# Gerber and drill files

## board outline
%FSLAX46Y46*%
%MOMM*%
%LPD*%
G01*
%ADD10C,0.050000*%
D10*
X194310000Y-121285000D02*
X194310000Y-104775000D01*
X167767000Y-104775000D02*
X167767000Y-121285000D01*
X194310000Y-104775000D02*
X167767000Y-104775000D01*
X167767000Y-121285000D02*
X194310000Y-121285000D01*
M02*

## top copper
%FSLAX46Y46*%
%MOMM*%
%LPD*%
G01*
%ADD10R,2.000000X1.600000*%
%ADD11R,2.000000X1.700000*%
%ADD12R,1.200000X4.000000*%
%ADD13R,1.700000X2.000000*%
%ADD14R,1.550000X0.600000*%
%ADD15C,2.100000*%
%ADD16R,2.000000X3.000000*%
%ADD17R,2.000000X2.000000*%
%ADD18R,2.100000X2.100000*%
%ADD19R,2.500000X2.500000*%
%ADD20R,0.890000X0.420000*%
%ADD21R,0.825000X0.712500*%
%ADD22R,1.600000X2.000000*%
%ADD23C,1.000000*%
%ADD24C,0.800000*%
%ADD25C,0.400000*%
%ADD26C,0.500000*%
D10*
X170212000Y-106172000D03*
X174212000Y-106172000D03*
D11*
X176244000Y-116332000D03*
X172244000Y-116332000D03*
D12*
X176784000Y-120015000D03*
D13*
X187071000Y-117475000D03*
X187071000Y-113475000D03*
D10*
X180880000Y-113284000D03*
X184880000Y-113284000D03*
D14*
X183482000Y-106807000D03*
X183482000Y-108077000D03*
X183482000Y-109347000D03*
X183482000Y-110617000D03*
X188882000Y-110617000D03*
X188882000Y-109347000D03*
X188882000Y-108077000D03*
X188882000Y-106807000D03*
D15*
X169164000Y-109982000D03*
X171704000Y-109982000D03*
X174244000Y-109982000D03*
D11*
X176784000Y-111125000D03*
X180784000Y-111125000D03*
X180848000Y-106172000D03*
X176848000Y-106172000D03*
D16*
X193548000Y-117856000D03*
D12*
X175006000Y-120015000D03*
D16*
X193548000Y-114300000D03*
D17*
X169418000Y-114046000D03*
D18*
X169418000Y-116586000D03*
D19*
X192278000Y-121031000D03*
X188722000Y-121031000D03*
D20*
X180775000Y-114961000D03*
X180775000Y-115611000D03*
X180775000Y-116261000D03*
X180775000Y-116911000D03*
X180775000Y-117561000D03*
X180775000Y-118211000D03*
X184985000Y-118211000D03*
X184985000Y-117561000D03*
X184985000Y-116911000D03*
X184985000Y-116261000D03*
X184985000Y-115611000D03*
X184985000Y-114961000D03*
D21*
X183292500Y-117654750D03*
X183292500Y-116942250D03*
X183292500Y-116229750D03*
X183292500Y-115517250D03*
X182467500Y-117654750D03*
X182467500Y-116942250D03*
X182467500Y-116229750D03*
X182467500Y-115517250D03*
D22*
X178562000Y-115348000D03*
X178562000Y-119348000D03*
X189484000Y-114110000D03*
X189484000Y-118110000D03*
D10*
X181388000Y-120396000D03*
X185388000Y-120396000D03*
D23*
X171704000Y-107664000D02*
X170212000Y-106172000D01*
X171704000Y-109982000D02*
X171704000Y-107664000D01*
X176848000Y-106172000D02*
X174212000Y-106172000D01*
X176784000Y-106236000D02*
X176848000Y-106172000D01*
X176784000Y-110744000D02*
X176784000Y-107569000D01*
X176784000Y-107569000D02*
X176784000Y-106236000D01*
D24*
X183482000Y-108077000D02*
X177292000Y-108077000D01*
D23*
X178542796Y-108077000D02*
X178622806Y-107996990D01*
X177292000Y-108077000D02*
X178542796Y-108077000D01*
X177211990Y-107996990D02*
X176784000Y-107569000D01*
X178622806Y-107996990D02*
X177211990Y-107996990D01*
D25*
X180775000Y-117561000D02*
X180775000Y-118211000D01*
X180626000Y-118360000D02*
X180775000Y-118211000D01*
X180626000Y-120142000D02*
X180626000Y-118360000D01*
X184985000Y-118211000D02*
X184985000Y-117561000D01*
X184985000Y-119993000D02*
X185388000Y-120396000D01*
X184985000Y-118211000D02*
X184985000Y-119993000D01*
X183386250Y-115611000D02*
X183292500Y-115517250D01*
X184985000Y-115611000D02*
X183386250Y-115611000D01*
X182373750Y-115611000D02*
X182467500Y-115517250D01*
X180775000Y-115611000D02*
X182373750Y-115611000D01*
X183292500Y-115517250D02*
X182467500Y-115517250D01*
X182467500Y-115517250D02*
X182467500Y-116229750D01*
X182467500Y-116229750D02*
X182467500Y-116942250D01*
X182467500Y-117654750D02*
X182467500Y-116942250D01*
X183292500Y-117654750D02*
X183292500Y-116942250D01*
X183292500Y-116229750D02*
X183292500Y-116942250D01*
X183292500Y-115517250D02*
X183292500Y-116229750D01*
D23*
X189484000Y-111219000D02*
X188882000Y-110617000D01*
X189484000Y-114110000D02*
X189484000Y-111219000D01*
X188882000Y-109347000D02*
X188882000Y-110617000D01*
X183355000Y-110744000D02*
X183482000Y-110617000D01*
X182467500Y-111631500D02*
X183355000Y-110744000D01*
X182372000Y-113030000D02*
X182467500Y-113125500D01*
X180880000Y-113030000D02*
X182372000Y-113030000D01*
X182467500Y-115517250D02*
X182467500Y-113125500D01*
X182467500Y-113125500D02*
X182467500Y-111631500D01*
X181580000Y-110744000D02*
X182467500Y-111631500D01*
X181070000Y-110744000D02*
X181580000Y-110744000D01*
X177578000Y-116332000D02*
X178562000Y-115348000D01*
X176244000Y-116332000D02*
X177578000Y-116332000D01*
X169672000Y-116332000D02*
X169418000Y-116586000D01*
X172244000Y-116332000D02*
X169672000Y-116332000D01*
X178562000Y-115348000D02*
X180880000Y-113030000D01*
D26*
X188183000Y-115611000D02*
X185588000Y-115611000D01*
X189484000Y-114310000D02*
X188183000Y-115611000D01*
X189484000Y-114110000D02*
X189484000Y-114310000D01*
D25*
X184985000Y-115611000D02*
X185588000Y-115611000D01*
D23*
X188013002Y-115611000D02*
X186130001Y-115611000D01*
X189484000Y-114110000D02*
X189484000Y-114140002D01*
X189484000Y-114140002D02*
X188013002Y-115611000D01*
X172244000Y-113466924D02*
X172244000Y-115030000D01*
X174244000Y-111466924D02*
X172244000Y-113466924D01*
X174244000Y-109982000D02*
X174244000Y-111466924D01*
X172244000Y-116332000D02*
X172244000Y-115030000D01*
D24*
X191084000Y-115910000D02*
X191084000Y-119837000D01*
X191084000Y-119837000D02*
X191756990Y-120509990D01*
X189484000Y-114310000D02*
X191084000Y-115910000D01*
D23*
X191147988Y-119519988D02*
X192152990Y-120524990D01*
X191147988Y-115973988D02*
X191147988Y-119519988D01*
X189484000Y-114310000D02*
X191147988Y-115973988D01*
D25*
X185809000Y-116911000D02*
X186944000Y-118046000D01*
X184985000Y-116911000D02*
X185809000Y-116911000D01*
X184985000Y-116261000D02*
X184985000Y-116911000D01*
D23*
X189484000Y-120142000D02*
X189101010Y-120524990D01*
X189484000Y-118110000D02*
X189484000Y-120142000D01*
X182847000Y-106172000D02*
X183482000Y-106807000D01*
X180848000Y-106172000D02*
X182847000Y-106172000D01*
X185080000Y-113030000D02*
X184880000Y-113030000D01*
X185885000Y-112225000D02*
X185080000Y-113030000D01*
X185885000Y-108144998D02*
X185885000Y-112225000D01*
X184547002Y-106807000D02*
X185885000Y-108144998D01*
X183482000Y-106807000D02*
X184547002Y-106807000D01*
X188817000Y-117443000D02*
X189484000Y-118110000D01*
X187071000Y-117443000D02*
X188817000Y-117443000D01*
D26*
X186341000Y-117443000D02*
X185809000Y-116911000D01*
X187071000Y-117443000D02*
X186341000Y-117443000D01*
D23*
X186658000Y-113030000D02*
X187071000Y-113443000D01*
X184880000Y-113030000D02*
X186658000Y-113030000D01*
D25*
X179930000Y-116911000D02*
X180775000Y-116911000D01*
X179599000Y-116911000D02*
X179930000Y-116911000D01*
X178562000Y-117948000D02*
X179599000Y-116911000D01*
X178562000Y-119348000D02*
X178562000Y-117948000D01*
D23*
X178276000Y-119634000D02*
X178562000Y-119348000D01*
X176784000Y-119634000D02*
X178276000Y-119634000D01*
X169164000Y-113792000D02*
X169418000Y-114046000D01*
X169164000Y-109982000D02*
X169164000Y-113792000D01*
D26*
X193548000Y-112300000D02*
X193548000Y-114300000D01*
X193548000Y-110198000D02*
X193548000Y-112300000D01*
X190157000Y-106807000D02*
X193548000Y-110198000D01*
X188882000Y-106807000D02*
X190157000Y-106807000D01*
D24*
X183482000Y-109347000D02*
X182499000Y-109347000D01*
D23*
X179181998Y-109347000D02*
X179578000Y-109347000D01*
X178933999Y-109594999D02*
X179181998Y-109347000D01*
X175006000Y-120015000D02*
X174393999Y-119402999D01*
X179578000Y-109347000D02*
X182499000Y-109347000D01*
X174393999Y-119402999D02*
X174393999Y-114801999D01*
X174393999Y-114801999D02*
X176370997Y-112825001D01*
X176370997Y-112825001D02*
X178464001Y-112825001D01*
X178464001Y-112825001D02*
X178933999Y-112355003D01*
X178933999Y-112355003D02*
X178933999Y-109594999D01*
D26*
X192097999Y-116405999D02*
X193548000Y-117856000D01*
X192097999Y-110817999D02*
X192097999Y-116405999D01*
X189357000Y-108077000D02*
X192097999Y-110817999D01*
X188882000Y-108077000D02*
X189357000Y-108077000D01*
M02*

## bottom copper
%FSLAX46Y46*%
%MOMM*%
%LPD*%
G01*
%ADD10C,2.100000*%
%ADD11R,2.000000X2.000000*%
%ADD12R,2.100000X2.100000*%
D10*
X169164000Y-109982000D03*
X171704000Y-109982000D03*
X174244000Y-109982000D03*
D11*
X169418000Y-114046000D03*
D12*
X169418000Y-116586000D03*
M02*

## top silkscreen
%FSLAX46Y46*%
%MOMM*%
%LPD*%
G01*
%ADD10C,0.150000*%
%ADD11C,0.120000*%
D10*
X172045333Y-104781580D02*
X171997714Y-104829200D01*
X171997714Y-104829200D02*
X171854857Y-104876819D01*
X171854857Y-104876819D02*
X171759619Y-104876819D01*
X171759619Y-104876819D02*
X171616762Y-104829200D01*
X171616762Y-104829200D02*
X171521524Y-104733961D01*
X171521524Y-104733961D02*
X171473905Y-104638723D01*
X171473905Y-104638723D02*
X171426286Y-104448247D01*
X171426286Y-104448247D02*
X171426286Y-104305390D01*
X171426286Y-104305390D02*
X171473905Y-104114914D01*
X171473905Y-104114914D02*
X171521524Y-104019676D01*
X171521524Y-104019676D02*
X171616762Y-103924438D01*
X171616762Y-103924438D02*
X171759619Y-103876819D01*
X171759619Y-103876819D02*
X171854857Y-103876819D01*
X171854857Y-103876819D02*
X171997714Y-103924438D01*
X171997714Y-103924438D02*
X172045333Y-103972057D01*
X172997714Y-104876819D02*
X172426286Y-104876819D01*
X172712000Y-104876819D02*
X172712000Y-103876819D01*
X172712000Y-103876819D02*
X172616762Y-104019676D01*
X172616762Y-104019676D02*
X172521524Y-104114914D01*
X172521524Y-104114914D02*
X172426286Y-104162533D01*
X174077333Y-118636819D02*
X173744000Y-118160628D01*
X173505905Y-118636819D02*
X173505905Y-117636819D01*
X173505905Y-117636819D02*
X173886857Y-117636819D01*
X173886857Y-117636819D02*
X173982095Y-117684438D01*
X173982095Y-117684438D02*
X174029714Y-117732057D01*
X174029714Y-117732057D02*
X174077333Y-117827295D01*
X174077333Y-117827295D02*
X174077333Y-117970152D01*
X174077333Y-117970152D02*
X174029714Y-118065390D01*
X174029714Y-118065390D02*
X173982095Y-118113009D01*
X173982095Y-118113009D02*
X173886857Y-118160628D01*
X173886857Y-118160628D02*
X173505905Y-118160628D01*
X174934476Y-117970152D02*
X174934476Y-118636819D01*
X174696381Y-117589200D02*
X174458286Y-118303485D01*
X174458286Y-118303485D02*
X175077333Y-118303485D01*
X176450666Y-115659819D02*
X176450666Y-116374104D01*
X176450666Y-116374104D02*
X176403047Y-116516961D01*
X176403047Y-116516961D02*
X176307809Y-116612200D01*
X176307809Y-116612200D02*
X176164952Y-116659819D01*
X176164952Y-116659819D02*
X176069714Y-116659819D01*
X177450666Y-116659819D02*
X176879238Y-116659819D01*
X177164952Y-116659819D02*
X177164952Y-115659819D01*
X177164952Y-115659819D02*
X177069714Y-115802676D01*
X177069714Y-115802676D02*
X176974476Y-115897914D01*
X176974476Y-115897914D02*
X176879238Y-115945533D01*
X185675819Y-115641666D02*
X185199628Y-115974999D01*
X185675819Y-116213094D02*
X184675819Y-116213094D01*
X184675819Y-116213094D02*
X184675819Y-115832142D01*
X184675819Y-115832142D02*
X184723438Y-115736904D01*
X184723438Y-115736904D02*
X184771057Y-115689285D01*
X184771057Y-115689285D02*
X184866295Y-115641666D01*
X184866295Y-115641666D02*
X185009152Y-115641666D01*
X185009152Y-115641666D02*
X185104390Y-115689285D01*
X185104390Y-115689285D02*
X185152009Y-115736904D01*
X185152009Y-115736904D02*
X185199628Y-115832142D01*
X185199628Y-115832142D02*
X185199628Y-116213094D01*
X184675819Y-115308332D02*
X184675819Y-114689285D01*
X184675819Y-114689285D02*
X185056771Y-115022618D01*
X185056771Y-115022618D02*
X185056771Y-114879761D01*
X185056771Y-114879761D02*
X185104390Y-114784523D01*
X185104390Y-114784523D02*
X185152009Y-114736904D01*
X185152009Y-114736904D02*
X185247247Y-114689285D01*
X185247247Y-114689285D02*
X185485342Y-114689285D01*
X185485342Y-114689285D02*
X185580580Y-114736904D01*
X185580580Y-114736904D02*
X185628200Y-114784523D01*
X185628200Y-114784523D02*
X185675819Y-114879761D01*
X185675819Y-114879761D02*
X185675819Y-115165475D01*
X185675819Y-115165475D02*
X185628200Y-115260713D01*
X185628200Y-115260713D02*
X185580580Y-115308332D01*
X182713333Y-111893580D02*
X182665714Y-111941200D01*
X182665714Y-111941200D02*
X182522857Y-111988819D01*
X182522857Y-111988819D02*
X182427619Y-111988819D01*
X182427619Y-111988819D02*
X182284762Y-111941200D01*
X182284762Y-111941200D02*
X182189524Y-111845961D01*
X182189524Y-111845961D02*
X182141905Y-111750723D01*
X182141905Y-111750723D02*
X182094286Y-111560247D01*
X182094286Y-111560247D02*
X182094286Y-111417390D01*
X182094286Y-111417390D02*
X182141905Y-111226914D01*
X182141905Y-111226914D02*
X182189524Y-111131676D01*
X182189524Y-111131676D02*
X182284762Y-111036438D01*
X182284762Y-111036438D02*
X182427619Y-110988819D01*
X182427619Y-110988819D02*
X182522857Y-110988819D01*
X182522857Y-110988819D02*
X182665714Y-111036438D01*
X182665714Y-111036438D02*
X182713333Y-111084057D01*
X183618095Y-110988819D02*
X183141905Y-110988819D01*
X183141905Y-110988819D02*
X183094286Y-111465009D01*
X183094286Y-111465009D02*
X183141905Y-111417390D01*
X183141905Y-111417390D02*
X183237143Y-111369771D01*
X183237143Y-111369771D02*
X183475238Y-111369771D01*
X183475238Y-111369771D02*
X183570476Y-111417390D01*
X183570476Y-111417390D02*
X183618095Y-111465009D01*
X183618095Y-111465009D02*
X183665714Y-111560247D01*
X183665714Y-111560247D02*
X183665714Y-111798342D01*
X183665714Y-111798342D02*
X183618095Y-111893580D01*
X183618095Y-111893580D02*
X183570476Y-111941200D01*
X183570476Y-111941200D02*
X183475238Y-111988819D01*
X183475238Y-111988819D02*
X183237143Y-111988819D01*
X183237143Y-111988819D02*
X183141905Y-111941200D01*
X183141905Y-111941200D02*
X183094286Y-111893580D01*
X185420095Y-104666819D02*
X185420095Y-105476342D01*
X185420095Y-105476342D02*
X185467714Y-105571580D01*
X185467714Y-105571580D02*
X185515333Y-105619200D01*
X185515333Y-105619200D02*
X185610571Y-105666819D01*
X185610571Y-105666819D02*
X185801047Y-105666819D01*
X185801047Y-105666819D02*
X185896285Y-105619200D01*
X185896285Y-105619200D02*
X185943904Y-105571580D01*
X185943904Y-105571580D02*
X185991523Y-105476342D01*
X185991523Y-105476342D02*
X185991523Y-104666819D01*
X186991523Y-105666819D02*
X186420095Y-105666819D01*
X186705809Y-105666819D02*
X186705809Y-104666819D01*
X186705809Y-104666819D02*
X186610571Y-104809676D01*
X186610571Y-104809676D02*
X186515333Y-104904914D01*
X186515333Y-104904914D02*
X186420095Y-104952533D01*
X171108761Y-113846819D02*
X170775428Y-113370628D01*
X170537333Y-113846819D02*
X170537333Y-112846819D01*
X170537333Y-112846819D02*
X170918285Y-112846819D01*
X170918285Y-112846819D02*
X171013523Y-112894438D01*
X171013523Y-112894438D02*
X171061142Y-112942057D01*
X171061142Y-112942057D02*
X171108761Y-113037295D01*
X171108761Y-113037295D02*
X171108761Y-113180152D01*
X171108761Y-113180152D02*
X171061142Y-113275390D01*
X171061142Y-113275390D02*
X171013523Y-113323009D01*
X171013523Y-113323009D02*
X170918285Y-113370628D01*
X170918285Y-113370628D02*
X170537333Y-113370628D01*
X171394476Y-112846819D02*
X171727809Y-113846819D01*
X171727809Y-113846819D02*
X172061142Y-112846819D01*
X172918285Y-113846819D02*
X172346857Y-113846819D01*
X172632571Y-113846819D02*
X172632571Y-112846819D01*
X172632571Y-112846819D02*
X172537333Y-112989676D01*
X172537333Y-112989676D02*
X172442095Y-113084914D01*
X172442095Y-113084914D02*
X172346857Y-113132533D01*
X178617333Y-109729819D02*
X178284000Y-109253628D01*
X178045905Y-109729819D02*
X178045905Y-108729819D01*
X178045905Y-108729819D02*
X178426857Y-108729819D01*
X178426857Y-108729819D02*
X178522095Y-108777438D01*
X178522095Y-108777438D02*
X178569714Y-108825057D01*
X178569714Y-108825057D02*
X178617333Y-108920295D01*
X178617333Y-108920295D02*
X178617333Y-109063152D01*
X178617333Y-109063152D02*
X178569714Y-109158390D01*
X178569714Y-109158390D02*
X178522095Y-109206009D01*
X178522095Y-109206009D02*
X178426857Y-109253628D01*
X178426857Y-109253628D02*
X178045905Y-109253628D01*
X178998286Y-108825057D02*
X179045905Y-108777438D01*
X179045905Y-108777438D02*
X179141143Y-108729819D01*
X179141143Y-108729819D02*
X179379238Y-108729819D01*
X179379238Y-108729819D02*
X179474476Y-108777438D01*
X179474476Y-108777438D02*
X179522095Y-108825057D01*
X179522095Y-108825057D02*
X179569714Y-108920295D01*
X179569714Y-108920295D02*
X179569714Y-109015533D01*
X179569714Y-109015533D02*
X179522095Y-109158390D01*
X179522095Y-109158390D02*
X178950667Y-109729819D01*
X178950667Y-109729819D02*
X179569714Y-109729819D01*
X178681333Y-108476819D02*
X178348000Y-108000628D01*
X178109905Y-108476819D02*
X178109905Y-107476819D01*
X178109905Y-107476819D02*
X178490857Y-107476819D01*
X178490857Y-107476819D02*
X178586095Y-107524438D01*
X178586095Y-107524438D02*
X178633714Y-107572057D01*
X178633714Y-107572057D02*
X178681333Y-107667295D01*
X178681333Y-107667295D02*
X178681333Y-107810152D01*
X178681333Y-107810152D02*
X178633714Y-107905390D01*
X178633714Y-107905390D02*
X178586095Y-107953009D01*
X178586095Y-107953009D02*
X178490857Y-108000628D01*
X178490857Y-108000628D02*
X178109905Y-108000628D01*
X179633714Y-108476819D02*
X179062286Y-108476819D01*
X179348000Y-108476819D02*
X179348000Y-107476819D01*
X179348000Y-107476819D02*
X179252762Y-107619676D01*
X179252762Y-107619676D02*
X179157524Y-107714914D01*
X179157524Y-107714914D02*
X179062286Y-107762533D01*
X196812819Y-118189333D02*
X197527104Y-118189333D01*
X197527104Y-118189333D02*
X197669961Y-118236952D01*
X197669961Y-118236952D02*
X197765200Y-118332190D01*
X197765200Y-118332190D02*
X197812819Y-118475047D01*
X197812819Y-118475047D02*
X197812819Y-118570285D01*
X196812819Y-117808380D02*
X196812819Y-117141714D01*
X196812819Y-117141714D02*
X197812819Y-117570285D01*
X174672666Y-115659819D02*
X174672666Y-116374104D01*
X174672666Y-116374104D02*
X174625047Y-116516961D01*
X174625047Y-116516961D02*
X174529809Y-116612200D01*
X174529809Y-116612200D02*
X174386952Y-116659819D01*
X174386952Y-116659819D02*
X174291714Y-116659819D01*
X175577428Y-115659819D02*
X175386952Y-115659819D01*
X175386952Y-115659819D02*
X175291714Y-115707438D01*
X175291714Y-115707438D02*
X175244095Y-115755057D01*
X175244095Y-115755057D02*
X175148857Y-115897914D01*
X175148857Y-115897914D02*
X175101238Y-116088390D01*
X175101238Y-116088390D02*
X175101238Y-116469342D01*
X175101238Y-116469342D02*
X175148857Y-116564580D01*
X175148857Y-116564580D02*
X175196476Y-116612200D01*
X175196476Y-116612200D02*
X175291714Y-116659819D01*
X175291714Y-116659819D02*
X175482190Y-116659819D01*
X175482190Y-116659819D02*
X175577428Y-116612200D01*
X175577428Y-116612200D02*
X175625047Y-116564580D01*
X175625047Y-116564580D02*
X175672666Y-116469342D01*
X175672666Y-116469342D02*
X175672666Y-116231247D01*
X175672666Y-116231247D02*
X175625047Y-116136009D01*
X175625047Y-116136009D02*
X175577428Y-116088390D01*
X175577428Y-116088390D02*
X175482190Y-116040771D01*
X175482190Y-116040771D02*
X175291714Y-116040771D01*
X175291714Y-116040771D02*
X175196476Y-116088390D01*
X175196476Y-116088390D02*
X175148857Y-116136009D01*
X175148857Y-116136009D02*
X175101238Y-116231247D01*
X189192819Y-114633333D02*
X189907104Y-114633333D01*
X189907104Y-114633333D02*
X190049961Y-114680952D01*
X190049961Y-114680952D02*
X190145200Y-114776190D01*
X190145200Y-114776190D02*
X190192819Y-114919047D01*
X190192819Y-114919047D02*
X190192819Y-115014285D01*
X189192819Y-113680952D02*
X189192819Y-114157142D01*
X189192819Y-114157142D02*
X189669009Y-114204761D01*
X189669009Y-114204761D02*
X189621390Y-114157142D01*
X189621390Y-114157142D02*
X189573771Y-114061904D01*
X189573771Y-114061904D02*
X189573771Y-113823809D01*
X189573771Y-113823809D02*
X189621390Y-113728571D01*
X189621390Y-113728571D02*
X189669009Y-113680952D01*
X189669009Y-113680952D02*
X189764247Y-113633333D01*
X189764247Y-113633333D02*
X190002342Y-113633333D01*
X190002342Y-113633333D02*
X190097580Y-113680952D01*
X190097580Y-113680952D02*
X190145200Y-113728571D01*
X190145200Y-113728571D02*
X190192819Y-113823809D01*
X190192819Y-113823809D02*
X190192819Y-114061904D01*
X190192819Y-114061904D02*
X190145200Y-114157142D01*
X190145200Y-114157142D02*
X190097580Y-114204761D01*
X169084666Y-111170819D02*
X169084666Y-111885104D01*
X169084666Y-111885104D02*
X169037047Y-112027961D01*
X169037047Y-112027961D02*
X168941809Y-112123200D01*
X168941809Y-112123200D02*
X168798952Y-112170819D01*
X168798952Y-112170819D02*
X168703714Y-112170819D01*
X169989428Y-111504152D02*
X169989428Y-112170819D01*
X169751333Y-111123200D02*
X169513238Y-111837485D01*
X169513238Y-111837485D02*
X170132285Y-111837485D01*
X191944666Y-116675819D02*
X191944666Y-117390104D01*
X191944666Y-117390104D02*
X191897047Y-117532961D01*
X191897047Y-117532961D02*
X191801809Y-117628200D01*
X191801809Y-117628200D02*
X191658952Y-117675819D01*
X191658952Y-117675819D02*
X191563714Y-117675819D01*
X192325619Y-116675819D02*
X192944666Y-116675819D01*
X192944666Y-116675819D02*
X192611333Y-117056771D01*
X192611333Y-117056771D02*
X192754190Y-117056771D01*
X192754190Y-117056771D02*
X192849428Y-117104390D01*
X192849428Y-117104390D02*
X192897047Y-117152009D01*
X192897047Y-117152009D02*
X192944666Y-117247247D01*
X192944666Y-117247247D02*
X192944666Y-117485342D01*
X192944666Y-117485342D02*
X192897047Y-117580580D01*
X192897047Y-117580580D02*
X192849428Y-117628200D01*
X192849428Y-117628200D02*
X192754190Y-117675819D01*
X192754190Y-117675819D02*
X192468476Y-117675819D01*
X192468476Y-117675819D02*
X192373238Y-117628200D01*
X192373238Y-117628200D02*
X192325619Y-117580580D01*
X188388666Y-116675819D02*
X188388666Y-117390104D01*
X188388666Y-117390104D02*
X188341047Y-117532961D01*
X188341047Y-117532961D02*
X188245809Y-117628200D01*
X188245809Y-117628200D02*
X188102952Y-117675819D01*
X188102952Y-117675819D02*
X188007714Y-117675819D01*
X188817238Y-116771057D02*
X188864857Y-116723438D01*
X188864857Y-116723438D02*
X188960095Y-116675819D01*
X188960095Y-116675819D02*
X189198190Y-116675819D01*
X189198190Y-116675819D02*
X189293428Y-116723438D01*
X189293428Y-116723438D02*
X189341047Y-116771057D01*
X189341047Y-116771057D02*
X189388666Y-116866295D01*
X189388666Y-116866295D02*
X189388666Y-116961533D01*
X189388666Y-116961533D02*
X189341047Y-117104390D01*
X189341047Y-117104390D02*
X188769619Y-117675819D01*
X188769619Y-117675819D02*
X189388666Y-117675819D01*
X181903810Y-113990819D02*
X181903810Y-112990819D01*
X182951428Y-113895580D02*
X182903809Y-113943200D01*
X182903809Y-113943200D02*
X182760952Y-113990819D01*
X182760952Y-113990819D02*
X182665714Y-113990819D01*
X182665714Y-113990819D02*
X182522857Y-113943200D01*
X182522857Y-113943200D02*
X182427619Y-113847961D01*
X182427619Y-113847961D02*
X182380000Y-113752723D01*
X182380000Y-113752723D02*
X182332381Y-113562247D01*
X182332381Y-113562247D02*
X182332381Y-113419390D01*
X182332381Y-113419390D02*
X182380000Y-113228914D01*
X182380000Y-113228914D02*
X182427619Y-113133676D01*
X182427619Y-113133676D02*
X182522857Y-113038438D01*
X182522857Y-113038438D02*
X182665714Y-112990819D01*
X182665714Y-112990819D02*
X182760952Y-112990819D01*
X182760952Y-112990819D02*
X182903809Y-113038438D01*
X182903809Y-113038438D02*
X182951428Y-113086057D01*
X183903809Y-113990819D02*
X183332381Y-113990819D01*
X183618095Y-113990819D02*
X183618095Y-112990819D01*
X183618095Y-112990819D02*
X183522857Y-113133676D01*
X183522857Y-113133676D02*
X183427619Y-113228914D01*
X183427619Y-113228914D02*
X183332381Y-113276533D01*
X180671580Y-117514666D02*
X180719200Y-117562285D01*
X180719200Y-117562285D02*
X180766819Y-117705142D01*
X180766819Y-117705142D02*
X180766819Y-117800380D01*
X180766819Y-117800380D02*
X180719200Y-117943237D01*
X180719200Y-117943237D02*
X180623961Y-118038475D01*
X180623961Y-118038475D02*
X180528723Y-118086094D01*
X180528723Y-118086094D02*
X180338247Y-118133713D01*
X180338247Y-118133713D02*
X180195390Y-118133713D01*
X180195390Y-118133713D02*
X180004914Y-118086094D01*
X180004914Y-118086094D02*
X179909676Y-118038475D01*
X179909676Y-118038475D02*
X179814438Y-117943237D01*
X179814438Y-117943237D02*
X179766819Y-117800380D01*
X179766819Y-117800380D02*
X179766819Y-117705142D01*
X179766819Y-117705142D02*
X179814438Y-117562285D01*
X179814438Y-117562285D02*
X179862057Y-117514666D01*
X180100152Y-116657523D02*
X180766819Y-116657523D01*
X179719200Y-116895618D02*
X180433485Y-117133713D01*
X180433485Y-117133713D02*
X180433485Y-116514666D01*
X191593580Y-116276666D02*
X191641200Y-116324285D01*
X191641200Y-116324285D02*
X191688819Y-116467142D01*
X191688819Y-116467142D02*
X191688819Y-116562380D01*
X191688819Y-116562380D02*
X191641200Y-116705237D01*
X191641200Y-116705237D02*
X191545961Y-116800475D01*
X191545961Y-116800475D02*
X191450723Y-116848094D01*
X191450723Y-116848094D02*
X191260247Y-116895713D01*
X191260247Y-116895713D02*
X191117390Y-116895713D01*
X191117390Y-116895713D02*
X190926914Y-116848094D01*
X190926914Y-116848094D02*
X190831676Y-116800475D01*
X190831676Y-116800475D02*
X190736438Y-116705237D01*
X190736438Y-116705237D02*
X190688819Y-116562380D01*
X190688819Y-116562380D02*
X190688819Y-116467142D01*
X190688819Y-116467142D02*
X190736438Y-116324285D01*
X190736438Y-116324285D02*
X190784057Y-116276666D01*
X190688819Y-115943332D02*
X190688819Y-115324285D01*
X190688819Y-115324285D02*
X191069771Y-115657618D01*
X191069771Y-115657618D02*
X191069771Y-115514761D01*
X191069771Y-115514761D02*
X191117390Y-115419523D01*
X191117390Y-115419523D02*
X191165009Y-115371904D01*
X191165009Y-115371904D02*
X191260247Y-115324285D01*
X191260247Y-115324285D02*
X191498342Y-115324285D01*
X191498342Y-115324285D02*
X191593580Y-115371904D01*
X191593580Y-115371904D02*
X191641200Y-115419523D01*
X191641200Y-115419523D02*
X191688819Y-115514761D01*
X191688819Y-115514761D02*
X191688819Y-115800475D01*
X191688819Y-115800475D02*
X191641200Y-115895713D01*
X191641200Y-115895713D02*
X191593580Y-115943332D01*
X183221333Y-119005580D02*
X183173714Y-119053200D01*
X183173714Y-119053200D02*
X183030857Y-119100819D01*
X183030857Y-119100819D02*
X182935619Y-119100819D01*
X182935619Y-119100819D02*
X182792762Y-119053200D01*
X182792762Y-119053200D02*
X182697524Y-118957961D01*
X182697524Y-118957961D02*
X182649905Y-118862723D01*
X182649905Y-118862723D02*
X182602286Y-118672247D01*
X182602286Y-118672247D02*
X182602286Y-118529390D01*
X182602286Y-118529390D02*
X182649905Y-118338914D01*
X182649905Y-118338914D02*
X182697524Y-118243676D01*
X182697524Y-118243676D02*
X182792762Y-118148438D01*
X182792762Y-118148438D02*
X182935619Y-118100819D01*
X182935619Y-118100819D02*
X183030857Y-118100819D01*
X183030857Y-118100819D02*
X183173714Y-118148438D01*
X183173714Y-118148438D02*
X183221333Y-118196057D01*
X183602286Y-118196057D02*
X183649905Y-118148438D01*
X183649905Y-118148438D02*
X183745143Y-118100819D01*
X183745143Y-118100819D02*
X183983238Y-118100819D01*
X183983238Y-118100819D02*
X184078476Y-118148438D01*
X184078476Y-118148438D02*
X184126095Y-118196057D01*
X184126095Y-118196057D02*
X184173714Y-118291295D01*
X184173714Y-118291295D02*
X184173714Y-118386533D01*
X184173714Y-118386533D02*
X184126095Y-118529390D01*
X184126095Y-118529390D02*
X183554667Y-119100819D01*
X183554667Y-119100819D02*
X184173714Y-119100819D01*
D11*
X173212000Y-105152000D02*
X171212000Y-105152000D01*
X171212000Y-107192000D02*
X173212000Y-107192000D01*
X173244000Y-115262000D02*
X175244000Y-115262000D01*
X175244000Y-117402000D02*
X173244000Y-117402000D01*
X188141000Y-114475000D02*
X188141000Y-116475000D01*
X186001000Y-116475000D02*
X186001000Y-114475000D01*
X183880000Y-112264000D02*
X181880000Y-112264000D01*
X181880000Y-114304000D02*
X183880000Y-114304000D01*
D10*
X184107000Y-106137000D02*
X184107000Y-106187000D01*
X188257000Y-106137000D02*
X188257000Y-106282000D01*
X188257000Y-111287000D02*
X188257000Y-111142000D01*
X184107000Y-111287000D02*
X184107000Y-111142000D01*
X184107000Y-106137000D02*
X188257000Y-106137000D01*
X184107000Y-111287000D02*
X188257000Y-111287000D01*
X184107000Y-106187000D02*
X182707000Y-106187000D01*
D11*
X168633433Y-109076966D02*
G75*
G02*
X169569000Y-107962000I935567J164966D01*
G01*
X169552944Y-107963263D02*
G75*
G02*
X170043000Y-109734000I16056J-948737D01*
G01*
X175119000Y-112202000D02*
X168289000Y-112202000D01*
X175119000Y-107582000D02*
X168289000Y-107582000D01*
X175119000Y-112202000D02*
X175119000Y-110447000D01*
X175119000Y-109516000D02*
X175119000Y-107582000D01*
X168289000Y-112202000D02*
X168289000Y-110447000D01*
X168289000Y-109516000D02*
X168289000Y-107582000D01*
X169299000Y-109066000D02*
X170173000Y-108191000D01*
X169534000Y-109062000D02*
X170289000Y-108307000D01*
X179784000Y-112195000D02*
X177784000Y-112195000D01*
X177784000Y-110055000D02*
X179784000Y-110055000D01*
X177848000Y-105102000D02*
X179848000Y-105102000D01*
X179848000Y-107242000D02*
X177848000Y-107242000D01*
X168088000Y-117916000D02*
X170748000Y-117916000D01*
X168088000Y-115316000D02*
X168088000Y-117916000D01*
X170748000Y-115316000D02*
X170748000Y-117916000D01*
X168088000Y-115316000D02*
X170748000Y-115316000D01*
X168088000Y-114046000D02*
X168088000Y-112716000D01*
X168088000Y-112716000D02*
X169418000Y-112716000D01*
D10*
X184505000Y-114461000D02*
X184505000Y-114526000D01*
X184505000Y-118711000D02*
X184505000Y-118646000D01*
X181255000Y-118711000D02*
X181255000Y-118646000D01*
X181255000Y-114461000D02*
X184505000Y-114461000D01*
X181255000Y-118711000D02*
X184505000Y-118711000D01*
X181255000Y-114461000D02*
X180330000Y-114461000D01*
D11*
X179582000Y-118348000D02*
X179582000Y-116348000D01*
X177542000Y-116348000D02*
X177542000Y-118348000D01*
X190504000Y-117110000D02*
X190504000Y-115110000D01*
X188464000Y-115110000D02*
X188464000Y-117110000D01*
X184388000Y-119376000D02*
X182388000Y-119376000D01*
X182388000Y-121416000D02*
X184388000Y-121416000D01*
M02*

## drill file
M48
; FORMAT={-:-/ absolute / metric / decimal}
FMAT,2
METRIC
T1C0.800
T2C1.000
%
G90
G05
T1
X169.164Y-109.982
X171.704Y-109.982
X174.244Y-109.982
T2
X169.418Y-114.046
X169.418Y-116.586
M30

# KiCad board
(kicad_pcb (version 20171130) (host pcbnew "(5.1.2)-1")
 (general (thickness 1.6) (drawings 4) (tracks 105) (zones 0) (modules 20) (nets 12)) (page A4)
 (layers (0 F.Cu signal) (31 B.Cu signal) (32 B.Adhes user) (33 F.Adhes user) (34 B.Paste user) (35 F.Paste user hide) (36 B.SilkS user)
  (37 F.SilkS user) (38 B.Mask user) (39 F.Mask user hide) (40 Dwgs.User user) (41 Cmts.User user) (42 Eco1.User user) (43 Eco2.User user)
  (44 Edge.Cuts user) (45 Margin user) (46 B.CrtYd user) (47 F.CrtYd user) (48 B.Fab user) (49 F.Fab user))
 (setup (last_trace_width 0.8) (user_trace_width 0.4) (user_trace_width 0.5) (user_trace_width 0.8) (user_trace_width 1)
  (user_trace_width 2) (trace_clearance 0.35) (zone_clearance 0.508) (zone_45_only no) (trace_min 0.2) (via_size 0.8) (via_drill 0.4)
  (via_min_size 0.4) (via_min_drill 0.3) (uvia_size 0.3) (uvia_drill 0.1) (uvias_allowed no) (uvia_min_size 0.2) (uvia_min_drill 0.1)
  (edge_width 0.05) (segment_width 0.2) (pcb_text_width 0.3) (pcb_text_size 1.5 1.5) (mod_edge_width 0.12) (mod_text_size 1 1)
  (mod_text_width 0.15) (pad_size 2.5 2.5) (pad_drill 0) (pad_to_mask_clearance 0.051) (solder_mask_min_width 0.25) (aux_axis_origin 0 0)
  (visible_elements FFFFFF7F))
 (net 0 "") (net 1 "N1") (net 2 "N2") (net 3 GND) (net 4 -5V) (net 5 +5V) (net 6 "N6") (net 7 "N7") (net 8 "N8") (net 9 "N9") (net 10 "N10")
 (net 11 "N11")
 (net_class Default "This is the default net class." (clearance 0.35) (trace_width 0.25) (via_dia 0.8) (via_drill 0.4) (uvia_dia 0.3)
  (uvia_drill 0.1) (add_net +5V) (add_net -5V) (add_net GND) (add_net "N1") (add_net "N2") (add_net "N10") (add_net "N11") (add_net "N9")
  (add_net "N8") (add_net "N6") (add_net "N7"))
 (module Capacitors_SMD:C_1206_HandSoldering (layer F.Cu) (at 172.212 106.172)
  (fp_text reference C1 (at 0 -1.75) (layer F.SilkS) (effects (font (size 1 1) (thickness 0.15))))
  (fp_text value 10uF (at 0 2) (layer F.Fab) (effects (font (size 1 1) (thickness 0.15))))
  (fp_line (start 1 -1.02) (end -1 -1.02) (layer F.SilkS) (width 0.12))
  (fp_line (start -1 1.02) (end 1 1.02) (layer F.SilkS) (width 0.12))
  (pad 1 smd rect (at -2 0) (size 2 1.6) (layers F.Cu F.Paste F.Mask) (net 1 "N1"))
  (pad 2 smd rect (at 2 0) (size 2 1.6) (layers F.Cu F.Paste F.Mask) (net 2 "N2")))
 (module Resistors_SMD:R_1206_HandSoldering (layer F.Cu) (at 174.244 116.332 180)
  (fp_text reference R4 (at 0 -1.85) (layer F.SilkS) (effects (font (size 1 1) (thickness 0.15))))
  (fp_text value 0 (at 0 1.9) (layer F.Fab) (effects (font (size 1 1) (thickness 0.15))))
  (fp_line (start 1 1.07) (end -1 1.07) (layer F.SilkS) (width 0.12))
  (fp_line (start -1 -1.07) (end 1 -1.07) (layer F.SilkS) (width 0.12))
  (pad 1 smd rect (at -2 0 180) (size 2 1.7) (layers F.Cu F.Paste F.Mask) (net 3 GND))
  (pad 2 smd rect (at 2 0 180) (size 2 1.7) (layers F.Cu F.Paste F.Mask) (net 3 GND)))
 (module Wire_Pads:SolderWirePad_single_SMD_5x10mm (layer F.Cu) (at 176.784 120.015)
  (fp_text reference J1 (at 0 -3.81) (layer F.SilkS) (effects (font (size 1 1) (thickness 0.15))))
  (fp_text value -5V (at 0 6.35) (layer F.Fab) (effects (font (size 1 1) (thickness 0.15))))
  (pad 1 smd rect (at 0 0) (size 1.2 4) (layers F.Cu F.Paste F.Mask) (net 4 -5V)))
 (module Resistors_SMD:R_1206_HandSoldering (layer F.Cu) (at 187.071 115.475 90)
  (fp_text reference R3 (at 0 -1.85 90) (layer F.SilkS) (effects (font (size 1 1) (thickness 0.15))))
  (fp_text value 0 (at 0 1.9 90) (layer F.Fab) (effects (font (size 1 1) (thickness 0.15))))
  (fp_line (start 1 1.07) (end -1 1.07) (layer F.SilkS) (width 0.12))
  (fp_line (start -1 -1.07) (end 1 -1.07) (layer F.SilkS) (width 0.12))
  (pad 1 smd rect (at -2 0 90) (size 2 1.7) (layers F.Cu F.Paste F.Mask) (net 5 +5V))
  (pad 2 smd rect (at 2 0 90) (size 2 1.7) (layers F.Cu F.Paste F.Mask) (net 5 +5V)))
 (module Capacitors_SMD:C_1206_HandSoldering (layer F.Cu) (at 182.88 113.284)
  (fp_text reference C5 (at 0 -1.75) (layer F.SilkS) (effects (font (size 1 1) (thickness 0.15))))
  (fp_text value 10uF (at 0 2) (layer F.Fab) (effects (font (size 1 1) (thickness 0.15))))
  (fp_line (start 1 -1.02) (end -1 -1.02) (layer F.SilkS) (width 0.12))
  (fp_line (start -1 1.02) (end 1 1.02) (layer F.SilkS) (width 0.12))
  (pad 1 smd rect (at -2 0) (size 2 1.6) (layers F.Cu F.Paste F.Mask) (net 3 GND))
  (pad 2 smd rect (at 2 0) (size 2 1.6) (layers F.Cu F.Paste F.Mask) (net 5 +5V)))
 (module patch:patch (layer F.Cu) (at 177.0888 111.5568)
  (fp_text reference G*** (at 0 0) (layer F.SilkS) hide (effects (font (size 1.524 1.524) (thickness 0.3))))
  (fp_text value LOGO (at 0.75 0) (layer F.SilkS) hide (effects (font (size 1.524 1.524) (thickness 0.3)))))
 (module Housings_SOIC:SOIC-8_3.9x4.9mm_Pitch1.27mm (layer F.Cu) (at 186.182 108.712)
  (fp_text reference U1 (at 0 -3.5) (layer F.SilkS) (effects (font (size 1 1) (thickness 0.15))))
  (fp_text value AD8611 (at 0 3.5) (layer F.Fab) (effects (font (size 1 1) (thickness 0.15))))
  (fp_line (start -2.075 -2.575) (end -2.075 -2.525) (layer F.SilkS) (width 0.15))
  (fp_line (start 2.075 -2.575) (end 2.075 -2.43) (layer F.SilkS) (width 0.15))
  (fp_line (start 2.075 2.575) (end 2.075 2.43) (layer F.SilkS) (width 0.15))
  (fp_line (start -2.075 2.575) (end -2.075 2.43) (layer F.SilkS) (width 0.15))
  (fp_line (start -2.075 -2.575) (end 2.075 -2.575) (layer F.SilkS) (width 0.15))
  (fp_line (start -2.075 2.575) (end 2.075 2.575) (layer F.SilkS) (width 0.15))
  (fp_line (start -2.075 -2.525) (end -3.475 -2.525) (layer F.SilkS) (width 0.15))
  (pad 1 smd rect (at -2.7 -1.905) (size 1.55 0.6) (layers F.Cu F.Paste F.Mask) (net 5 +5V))
  (pad 2 smd rect (at -2.7 -0.635) (size 1.55 0.6) (layers F.Cu F.Paste F.Mask) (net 2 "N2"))
  (pad 3 smd rect (at -2.7 0.635) (size 1.55 0.6) (layers F.Cu F.Paste F.Mask) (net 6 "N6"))
  (pad 4 smd rect (at -2.7 1.905) (size 1.55 0.6) (layers F.Cu F.Paste F.Mask) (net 3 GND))
  (pad 5 smd rect (at 2.7 1.905) (size 1.55 0.6) (layers F.Cu F.Paste F.Mask) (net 3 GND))
  (pad 6 smd rect (at 2.7 0.635) (size 1.55 0.6) (layers F.Cu F.Paste F.Mask) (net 3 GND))
  (pad 7 smd rect (at 2.7 -0.635) (size 1.55 0.6) (layers F.Cu F.Paste F.Mask) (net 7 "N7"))
  (pad 8 smd rect (at 2.7 -1.905) (size 1.55 0.6) (layers F.Cu F.Paste F.Mask) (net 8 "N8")))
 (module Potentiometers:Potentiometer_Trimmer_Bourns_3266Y (layer F.Cu) (at 169.164 109.982 180)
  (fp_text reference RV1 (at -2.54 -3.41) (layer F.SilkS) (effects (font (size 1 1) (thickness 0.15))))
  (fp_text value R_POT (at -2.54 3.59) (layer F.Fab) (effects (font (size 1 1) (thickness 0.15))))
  (fp_arc (start -0.405 1.07) (end -0.405 2.02) (angle -100) (layer F.SilkS) (width 0.12))
  (fp_arc (start -0.405 1.07) (end -0.879 0.248) (angle -151) (layer F.SilkS) (width 0.12))
  (fp_line (start -5.955 -2.22) (end 0.875 -2.22) (layer F.SilkS) (width 0.12))
  (fp_line (start -5.955 2.4) (end 0.875 2.4) (layer F.SilkS) (width 0.12))
  (fp_line (start -5.955 -2.22) (end -5.955 -0.465) (layer F.SilkS) (width 0.12))
  (fp_line (start -5.955 0.466) (end -5.955 2.4) (layer F.SilkS) (width 0.12))
  (fp_line (start 0.875 -2.22) (end 0.875 -0.465) (layer F.SilkS) (width 0.12))
  (fp_line (start 0.875 0.466) (end 0.875 2.4) (layer F.SilkS) (width 0.12))
  (fp_line (start -0.135 0.916) (end -1.009 1.791) (layer F.SilkS) (width 0.12))
  (fp_line (start -0.37 0.92) (end -1.125 1.675) (layer F.SilkS) (width 0.12))
  (pad 1 thru_hole circle (at 0 0 180) (size 2.1 2.1) (drill 0.8) (layers *.Cu *.Mask) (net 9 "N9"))
  (pad 2 thru_hole circle (at -2.54 0 180) (size 2.1 2.1) (drill 0.8) (layers *.Cu *.Mask) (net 1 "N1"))
  (pad 3 thru_hole circle (at -5.08 0 180) (size 2.1 2.1) (drill 0.8) (layers *.Cu *.Mask) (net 3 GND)))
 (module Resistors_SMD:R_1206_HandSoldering (layer F.Cu) (at 178.784 111.125)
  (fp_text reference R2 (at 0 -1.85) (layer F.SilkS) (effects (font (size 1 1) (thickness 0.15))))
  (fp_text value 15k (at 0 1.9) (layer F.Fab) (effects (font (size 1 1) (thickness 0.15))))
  (fp_line (start 1 1.07) (end -1 1.07) (layer F.SilkS) (width 0.12))
  (fp_line (start -1 -1.07) (end 1 -1.07) (layer F.SilkS) (width 0.12))
  (pad 1 smd rect (at -2 0) (size 2 1.7) (layers F.Cu F.Paste F.Mask) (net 2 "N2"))
  (pad 2 smd rect (at 2 0) (size 2 1.7) (layers F.Cu F.Paste F.Mask) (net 3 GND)))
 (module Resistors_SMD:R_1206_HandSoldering (layer F.Cu) (at 178.848 106.172 180)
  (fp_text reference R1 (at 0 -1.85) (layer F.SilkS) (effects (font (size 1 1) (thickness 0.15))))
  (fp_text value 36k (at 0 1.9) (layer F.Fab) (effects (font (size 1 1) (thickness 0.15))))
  (fp_line (start 1 1.07) (end -1 1.07) (layer F.SilkS) (width 0.12))
  (fp_line (start -1 -1.07) (end 1 -1.07) (layer F.SilkS) (width 0.12))
  (pad 1 smd rect (at -2 0 180) (size 2 1.7) (layers F.Cu F.Paste F.Mask) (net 5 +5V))
  (pad 2 smd rect (at 2 0 180) (size 2 1.7) (layers F.Cu F.Paste F.Mask) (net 2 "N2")))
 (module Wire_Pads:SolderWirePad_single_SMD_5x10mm (layer F.Cu) (at 193.548 117.856 270)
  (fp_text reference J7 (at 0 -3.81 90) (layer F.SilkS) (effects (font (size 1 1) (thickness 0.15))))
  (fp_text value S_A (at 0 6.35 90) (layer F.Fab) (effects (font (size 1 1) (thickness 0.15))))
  (pad 1 smd rect (at 0 0 270) (size 3 2) (layers F.Cu F.Paste F.Mask) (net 7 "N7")))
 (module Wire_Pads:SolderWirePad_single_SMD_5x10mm (layer F.Cu) (at 175.006 120.015)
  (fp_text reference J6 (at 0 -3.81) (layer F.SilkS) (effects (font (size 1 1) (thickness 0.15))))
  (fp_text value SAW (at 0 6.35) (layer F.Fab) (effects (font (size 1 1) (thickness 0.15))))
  (pad 1 smd rect (at 0 0) (size 1.2 4) (layers F.Cu F.Paste F.Mask) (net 6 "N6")))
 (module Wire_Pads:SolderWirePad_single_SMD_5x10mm (layer F.Cu) (at 193.548 114.3 90)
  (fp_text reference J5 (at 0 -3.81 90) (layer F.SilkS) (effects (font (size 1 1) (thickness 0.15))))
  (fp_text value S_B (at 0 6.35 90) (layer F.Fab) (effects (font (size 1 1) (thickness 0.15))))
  (pad 1 smd rect (at 0 0 90) (size 3 2) (layers F.Cu F.Paste F.Mask) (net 8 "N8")))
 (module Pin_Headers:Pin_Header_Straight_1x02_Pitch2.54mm (layer F.Cu) (at 169.418 114.046)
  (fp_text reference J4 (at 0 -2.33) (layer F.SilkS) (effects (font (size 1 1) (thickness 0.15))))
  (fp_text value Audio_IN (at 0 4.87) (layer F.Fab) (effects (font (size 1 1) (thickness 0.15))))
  (fp_line (start -1.33 3.87) (end 1.33 3.87) (layer F.SilkS) (width 0.12))
  (fp_line (start -1.33 1.27) (end -1.33 3.87) (layer F.SilkS) (width 0.12))
  (fp_line (start 1.33 1.27) (end 1.33 3.87) (layer F.SilkS) (width 0.12))
  (fp_line (start -1.33 1.27) (end 1.33 1.27) (layer F.SilkS) (width 0.12))
  (fp_line (start -1.33 0) (end -1.33 -1.33) (layer F.SilkS) (width 0.12))
  (fp_line (start -1.33 -1.33) (end 0 -1.33) (layer F.SilkS) (width 0.12))
  (pad 1 thru_hole rect (at 0 0) (size 2 2) (drill 1) (layers *.Cu *.Mask) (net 9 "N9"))
  (pad 2 thru_hole rect (at 0 2.54) (size 2.1 2.1) (drill 1) (layers *.Cu *.Mask) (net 3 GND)))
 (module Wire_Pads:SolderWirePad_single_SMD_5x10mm (layer F.Cu) (at 192.278 121.031)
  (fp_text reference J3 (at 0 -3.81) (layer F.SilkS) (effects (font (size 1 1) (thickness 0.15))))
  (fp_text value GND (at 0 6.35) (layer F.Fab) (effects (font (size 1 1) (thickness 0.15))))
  (pad 1 smd rect (at 0 0) (size 2.5 2.5) (layers F.Cu F.Paste F.Mask) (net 3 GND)))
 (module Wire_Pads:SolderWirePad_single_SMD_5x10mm (layer F.Cu) (at 188.722 121.031)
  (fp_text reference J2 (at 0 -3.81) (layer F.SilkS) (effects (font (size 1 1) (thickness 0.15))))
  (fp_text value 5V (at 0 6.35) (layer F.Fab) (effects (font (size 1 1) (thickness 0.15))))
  (pad 1 smd rect (at 0 0) (size 2.5 2.5) (layers F.Cu F.Paste F.Mask) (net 5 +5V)))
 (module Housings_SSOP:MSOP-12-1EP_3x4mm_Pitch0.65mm (layer F.Cu) (at 182.88 116.586)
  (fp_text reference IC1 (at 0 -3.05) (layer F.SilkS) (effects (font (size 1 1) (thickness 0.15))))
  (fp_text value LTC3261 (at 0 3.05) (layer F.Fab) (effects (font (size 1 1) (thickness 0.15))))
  (fp_line (start 1.625 -2.125) (end 1.625 -2.06) (layer F.SilkS) (width 0.15))
  (fp_line (start 1.625 2.125) (end 1.625 2.06) (layer F.SilkS) (width 0.15))
  (fp_line (start -1.625 2.125) (end -1.625 2.06) (layer F.SilkS) (width 0.15))
  (fp_line (start -1.625 -2.125) (end 1.625 -2.125) (layer F.SilkS) (width 0.15))
  (fp_line (start -1.625 2.125) (end 1.625 2.125) (layer F.SilkS) (width 0.15))
  (fp_line (start -1.625 -2.125) (end -2.55 -2.125) (layer F.SilkS) (width 0.15))
  (pad 1 smd rect (at -2.105 -1.625) (size 0.89 0.42) (layers F.Cu F.Paste F.Mask))
  (pad 2 smd rect (at -2.105 -0.975) (size 0.89 0.42) (layers F.Cu F.Paste F.Mask) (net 3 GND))
  (pad 3 smd rect (at -2.105 -0.325) (size 0.89 0.42) (layers F.Cu F.Paste F.Mask))
  (pad 4 smd rect (at -2.105 0.325) (size 0.89 0.42) (layers F.Cu F.Paste F.Mask) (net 4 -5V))
  (pad 5 smd rect (at -2.105 0.975) (size 0.89 0.42) (layers F.Cu F.Paste F.Mask) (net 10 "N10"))
  (pad 6 smd rect (at -2.105 1.625) (size 0.89 0.42) (layers F.Cu F.Paste F.Mask) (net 10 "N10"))
  (pad 7 smd rect (at 2.105 1.625) (size 0.89 0.42) (layers F.Cu F.Paste F.Mask) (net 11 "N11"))
  (pad 8 smd rect (at 2.105 0.975) (size 0.89 0.42) (layers F.Cu F.Paste F.Mask) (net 11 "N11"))
  (pad 9 smd rect (at 2.105 0.325) (size 0.89 0.42) (layers F.Cu F.Paste F.Mask) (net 5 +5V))
  (pad 10 smd rect (at 2.105 -0.325) (size 0.89 0.42) (layers F.Cu F.Paste F.Mask) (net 5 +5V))
  (pad 11 smd rect (at 2.105 -0.975) (size 0.89 0.42) (layers F.Cu F.Paste F.Mask) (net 3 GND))
  (pad 12 smd rect (at 2.105 -1.625) (size 0.89 0.42) (layers F.Cu F.Paste F.Mask))
  (pad 13 smd rect (at 0.4125 1.06875) (size 0.825 0.7125) (layers F.Cu F.Paste F.Mask) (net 3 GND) (solder_paste_margin_ratio -0.2))
  (pad 13 smd rect (at 0.4125 0.35625) (size 0.825 0.7125) (layers F.Cu F.Paste F.Mask) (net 3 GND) (solder_paste_margin_ratio -0.2))
  (pad 13 smd rect (at 0.4125 -0.35625) (size 0.825 0.7125) (layers F.Cu F.Paste F.Mask) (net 3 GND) (solder_paste_margin_ratio -0.2))
  (pad 13 smd rect (at 0.4125 -1.06875) (size 0.825 0.7125) (layers F.Cu F.Paste F.Mask) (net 3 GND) (solder_paste_margin_ratio -0.2))
  (pad 13 smd rect (at -0.4125 1.06875) (size 0.825 0.7125) (layers F.Cu F.Paste F.Mask) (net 3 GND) (solder_paste_margin_ratio -0.2))
  (pad 13 smd rect (at -0.4125 0.35625) (size 0.825 0.7125) (layers F.Cu F.Paste F.Mask) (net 3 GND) (solder_paste_margin_ratio -0.2))
  (pad 13 smd rect (at -0.4125 -0.35625) (size 0.825 0.7125) (layers F.Cu F.Paste F.Mask) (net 3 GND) (solder_paste_margin_ratio -0.2))
  (pad 13 smd rect (at -0.4125 -1.06875) (size 0.825 0.7125) (layers F.Cu F.Paste F.Mask) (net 3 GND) (solder_paste_margin_ratio -0.2)))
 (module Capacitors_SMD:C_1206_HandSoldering (layer F.Cu) (at 178.562 117.348 270)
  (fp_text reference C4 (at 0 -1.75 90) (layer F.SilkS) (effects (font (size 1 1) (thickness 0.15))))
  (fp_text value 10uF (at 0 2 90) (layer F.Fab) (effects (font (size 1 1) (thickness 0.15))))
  (fp_line (start 1 -1.02) (end -1 -1.02) (layer F.SilkS) (width 0.12))
  (fp_line (start -1 1.02) (end 1 1.02) (layer F.SilkS) (width 0.12))
  (pad 1 smd rect (at -2 0 270) (size 2 1.6) (layers F.Cu F.Paste F.Mask) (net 3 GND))
  (pad 2 smd rect (at 2 0 270) (size 2 1.6) (layers F.Cu F.Paste F.Mask) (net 4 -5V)))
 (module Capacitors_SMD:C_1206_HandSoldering (layer F.Cu) (at 189.484 116.11 270)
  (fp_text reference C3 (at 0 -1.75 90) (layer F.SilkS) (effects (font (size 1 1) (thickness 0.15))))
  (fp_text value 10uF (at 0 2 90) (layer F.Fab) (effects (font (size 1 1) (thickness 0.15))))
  (fp_line (start 1 -1.02) (end -1 -1.02) (layer F.SilkS) (width 0.12))
  (fp_line (start -1 1.02) (end 1 1.02) (layer F.SilkS) (width 0.12))
  (pad 1 smd rect (at -2 0 270) (size 2 1.6) (layers F.Cu F.Paste F.Mask) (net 3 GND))
  (pad 2 smd rect (at 2 0 270) (size 2 1.6) (layers F.Cu F.Paste F.Mask) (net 5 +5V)))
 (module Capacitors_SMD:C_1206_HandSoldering (layer F.Cu) (at 183.388 120.396)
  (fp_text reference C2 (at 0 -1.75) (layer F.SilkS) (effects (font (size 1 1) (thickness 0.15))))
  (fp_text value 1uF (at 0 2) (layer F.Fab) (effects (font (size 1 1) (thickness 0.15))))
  (fp_line (start 1 -1.02) (end -1 -1.02) (layer F.SilkS) (width 0.12))
  (fp_line (start -1 1.02) (end 1 1.02) (layer F.SilkS) (width 0.12))
  (pad 1 smd rect (at -2 0) (size 2 1.6) (layers F.Cu F.Paste F.Mask) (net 10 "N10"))
  (pad 2 smd rect (at 2 0) (size 2 1.6) (layers F.Cu F.Paste F.Mask) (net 11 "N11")))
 (gr_line (start 194.31 121.285) (end 194.31 104.775) (layer Edge.Cuts) (width 0.05))
 (gr_line (start 167.767 104.775) (end 167.767 121.285) (layer Edge.Cuts) (width 0.05))
 (gr_line (start 194.31 104.775) (end 167.767 104.775) (layer Edge.Cuts) (width 0.05))
 (gr_line (start 167.767 121.285) (end 194.31 121.285) (layer Edge.Cuts) (width 0.05))
 (segment (start 171.704 107.664) (end 170.212 106.172) (width 1) (layer F.Cu) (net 1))
 (segment (start 171.704 109.982) (end 171.704 107.664) (width 1) (layer F.Cu) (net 1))
 (segment (start 176.848 106.172) (end 174.212 106.172) (width 1) (layer F.Cu) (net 2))
 (segment (start 176.784 106.236) (end 176.848 106.172) (width 1) (layer F.Cu) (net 2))
 (segment (start 176.784 110.744) (end 176.784 107.569) (width 1) (layer F.Cu) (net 2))
 (segment (start 176.784 107.569) (end 176.784 106.236) (width 1) (layer F.Cu) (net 2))
 (segment (start 183.482 108.077) (end 177.292 108.077) (width 0.8) (layer F.Cu) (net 2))
 (segment (start 178.542796 108.077) (end 178.622806 107.99699) (width 1) (layer F.Cu) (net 2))
 (segment (start 177.292 108.077) (end 178.542796 108.077) (width 1) (layer F.Cu) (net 2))
 (segment (start 177.21199 107.99699) (end 176.784 107.569) (width 1) (layer F.Cu) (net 2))
 (segment (start 178.622806 107.99699) (end 177.21199 107.99699) (width 1) (layer F.Cu) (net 2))
 (segment (start 180.775 117.561) (end 180.775 118.211) (width 0.4) (layer F.Cu) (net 10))
 (segment (start 180.626 118.36) (end 180.775 118.211) (width 0.4) (layer F.Cu) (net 10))
 (segment (start 180.626 120.142) (end 180.626 118.36) (width 0.4) (layer F.Cu) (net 10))
 (segment (start 184.985 118.211) (end 184.985 117.561) (width 0.4) (layer F.Cu) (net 11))
 (segment (start 184.985 119.993) (end 185.388 120.396) (width 0.4) (layer F.Cu) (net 11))
 (segment (start 184.985 118.211) (end 184.985 119.993) (width 0.4) (layer F.Cu) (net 11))
 (segment (start 183.38625 115.611) (end 183.2925 115.51725) (width 0.4) (layer F.Cu) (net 3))
 (segment (start 184.985 115.611) (end 183.38625 115.611) (width 0.4) (layer F.Cu) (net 3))
 (segment (start 182.37375 115.611) (end 182.4675 115.51725) (width 0.4) (layer F.Cu) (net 3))
 (segment (start 180.775 115.611) (end 182.37375 115.611) (width 0.4) (layer F.Cu) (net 3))
 (segment (start 183.2925 115.51725) (end 182.4675 115.51725) (width 0.4) (layer F.Cu) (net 3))
 (segment (start 182.4675 115.51725) (end 182.4675 116.22975) (width 0.4) (layer F.Cu) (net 3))
 (segment (start 182.4675 116.22975) (end 182.4675 116.94225) (width 0.4) (layer F.Cu) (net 3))
 (segment (start 182.4675 117.65475) (end 182.4675 116.94225) (width 0.4) (layer F.Cu) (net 3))
 (segment (start 183.2925 117.65475) (end 183.2925 116.94225) (width 0.4) (layer F.Cu) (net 3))
 (segment (start 183.2925 116.22975) (end 183.2925 116.94225) (width 0.4) (layer F.Cu) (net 3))
 (segment (start 183.2925 115.51725) (end 183.2925 116.22975) (width 0.4) (layer F.Cu) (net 3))
 (segment (start 189.484 111.219) (end 188.882 110.617) (width 1) (layer F.Cu) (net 3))
 (segment (start 189.484 114.11) (end 189.484 111.219) (width 1) (layer F.Cu) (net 3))
 (segment (start 188.882 109.347) (end 188.882 110.617) (width 1) (layer F.Cu) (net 3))
 (segment (start 183.355 110.744) (end 183.482 110.617) (width 1) (layer F.Cu) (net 3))
 (segment (start 182.4675 111.6315) (end 183.355 110.744) (width 1) (layer F.Cu) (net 3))
 (segment (start 182.372 113.03) (end 182.4675 113.1255) (width 1) (layer F.Cu) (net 3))
 (segment (start 180.88 113.03) (end 182.372 113.03) (width 1) (layer F.Cu) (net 3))
 (segment (start 182.4675 115.51725) (end 182.4675 113.1255) (width 1) (layer F.Cu) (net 3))
 (segment (start 182.4675 113.1255) (end 182.4675 111.6315) (width 1) (layer F.Cu) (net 3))
 (segment (start 181.58 110.744) (end 182.4675 111.6315) (width 1) (layer F.Cu) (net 3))
 (segment (start 181.07 110.744) (end 181.58 110.744) (width 1) (layer F.Cu) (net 3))
 (segment (start 177.578 116.332) (end 178.562 115.348) (width 1) (layer F.Cu) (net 3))
 (segment (start 176.244 116.332) (end 177.578 116.332) (width 1) (layer F.Cu) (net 3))
 (segment (start 169.672 116.332) (end 169.418 116.586) (width 1) (layer F.Cu) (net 3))
 (segment (start 172.244 116.332) (end 169.672 116.332) (width 1) (layer F.Cu) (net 3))
 (segment (start 178.562 115.348) (end 180.88 113.03) (width 1) (layer F.Cu) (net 3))
 (segment (start 188.183 115.611) (end 185.588 115.611) (width 0.5) (layer F.Cu) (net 3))
 (segment (start 189.484 114.31) (end 188.183 115.611) (width 0.5) (layer F.Cu) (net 3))
 (segment (start 189.484 114.11) (end 189.484 114.31) (width 0.5) (layer F.Cu) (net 3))
 (segment (start 184.985 115.611) (end 185.588 115.611) (width 0.4) (layer F.Cu) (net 3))
 (segment (start 188.013002 115.611) (end 186.130001 115.611) (width 1) (layer F.Cu) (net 3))
 (segment (start 189.484 114.11) (end 189.484 114.140002) (width 1) (layer F.Cu) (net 3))
 (segment (start 189.484 114.140002) (end 188.013002 115.611) (width 1) (layer F.Cu) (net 3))
 (segment (start 172.244 113.466924) (end 172.244 115.03) (width 1) (layer F.Cu) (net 3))
 (segment (start 174.244 111.466924) (end 172.244 113.466924) (width 1) (layer F.Cu) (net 3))
 (segment (start 174.244 109.982) (end 174.244 111.466924) (width 1) (layer F.Cu) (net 3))
 (segment (start 172.244 116.332) (end 172.244 115.03) (width 1) (layer F.Cu) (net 3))
 (segment (start 191.084 115.91) (end 191.084 119.837) (width 0.8) (layer F.Cu) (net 3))
 (segment (start 191.084 119.837) (end 191.75699 120.50999) (width 0.8) (layer F.Cu) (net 3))
 (segment (start 189.484 114.31) (end 191.084 115.91) (width 0.8) (layer F.Cu) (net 3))
 (segment (start 191.147988 119.519988) (end 192.15299 120.52499) (width 1) (layer F.Cu) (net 3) (status 1000000))
 (segment (start 191.147988 115.973988) (end 191.147988 119.519988) (width 1) (layer F.Cu) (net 3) (status 1000000))
 (segment (start 189.484 114.31) (end 191.147988 115.973988) (width 1) (layer F.Cu) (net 3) (status 1000000))
 (segment (start 185.809 116.911) (end 186.944 118.046) (width 0.4) (layer F.Cu) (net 5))
 (segment (start 184.985 116.911) (end 185.809 116.911) (width 0.4) (layer F.Cu) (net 5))
 (segment (start 184.985 116.261) (end 184.985 116.911) (width 0.4) (layer F.Cu) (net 5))
 (segment (start 189.484 120.142) (end 189.10101 120.52499) (width 1) (layer F.Cu) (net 5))
 (segment (start 189.484 118.11) (end 189.484 120.142) (width 1) (layer F.Cu) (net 5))
 (segment (start 182.847 106.172) (end 183.482 106.807) (width 1) (layer F.Cu) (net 5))
 (segment (start 180.848 106.172) (end 182.847 106.172) (width 1) (layer F.Cu) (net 5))
 (segment (start 185.08 113.03) (end 184.88 113.03) (width 1) (layer F.Cu) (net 5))
 (segment (start 185.885 112.225) (end 185.08 113.03) (width 1) (layer F.Cu) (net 5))
 (segment (start 185.885 108.144998) (end 185.885 112.225) (width 1) (layer F.Cu) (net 5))
 (segment (start 184.547002 106.807) (end 185.885 108.144998) (width 1) (layer F.Cu) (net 5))
 (segment (start 183.482 106.807) (end 184.547002 106.807) (width 1) (layer F.Cu) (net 5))
 (segment (start 188.817 117.443) (end 189.484 118.11) (width 1) (layer F.Cu) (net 5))
 (segment (start 187.071 117.443) (end 188.817 117.443) (width 1) (layer F.Cu) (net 5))
 (segment (start 186.341 117.443) (end 185.809 116.911) (width 0.5) (layer F.Cu) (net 5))
 (segment (start 187.071 117.443) (end 186.341 117.443) (width 0.5) (layer F.Cu) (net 5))
 (segment (start 186.658 113.03) (end 187.071 113.443) (width 1) (layer F.Cu) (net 5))
 (segment (start 184.88 113.03) (end 186.658 113.03) (width 1) (layer F.Cu) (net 5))
 (segment (start 179.93 116.911) (end 180.775 116.911) (width 0.4) (layer F.Cu) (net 4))
 (segment (start 179.599 116.911) (end 179.93 116.911) (width 0.4) (layer F.Cu) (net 4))
 (segment (start 178.562 117.948) (end 179.599 116.911) (width 0.4) (layer F.Cu) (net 4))
 (segment (start 178.562 119.348) (end 178.562 117.948) (width 0.4) (layer F.Cu) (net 4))
 (segment (start 178.276 119.634) (end 178.562 119.348) (width 1) (layer F.Cu) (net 4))
 (segment (start 176.784 119.634) (end 178.276 119.634) (width 1) (layer F.Cu) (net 4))
 (segment (start 169.164 113.792) (end 169.418 114.046) (width 1) (layer F.Cu) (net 9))
 (segment (start 169.164 109.982) (end 169.164 113.792) (width 1) (layer F.Cu) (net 9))
 (segment (start 193.548 112.3) (end 193.548 114.3) (width 0.5) (layer F.Cu) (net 8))
 (segment (start 193.548 110.198) (end 193.548 112.3) (width 0.5) (layer F.Cu) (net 8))
 (segment (start 190.157 106.807) (end 193.548 110.198) (width 0.5) (layer F.Cu) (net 8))
 (segment (start 188.882 106.807) (end 190.157 106.807) (width 0.5) (layer F.Cu) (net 8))
 (segment (start 183.482 109.347) (end 182.499 109.347) (width 0.8) (layer F.Cu) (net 6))
 (segment (start 179.181998 109.347) (end 179.578 109.347) (width 1) (layer F.Cu) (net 6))
 (segment (start 178.933999 109.594999) (end 179.181998 109.347) (width 1) (layer F.Cu) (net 6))
 (segment (start 175.006 120.015) (end 174.393999 119.402999) (width 1) (layer F.Cu) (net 6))
 (segment (start 179.578 109.347) (end 182.499 109.347) (width 1) (layer F.Cu) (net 6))
 (segment (start 174.393999 119.402999) (end 174.393999 114.801999) (width 1) (layer F.Cu) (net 6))
 (segment (start 174.393999 114.801999) (end 176.370997 112.825001) (width 1) (layer F.Cu) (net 6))
 (segment (start 176.370997 112.825001) (end 178.464001 112.825001) (width 1) (layer F.Cu) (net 6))
 (segment (start 178.464001 112.825001) (end 178.933999 112.355003) (width 1) (layer F.Cu) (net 6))
 (segment (start 178.933999 112.355003) (end 178.933999 109.594999) (width 1) (layer F.Cu) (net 6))
 (segment (start 192.097999 116.405999) (end 193.548 117.856) (width 0.5) (layer F.Cu) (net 7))
 (segment (start 192.097999 110.817999) (end 192.097999 116.405999) (width 0.5) (layer F.Cu) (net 7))
 (segment (start 189.357 108.077) (end 192.097999 110.817999) (width 0.5) (layer F.Cu) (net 7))
 (segment (start 188.882 108.077) (end 189.357 108.077) (width 0.5) (layer F.Cu) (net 7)))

